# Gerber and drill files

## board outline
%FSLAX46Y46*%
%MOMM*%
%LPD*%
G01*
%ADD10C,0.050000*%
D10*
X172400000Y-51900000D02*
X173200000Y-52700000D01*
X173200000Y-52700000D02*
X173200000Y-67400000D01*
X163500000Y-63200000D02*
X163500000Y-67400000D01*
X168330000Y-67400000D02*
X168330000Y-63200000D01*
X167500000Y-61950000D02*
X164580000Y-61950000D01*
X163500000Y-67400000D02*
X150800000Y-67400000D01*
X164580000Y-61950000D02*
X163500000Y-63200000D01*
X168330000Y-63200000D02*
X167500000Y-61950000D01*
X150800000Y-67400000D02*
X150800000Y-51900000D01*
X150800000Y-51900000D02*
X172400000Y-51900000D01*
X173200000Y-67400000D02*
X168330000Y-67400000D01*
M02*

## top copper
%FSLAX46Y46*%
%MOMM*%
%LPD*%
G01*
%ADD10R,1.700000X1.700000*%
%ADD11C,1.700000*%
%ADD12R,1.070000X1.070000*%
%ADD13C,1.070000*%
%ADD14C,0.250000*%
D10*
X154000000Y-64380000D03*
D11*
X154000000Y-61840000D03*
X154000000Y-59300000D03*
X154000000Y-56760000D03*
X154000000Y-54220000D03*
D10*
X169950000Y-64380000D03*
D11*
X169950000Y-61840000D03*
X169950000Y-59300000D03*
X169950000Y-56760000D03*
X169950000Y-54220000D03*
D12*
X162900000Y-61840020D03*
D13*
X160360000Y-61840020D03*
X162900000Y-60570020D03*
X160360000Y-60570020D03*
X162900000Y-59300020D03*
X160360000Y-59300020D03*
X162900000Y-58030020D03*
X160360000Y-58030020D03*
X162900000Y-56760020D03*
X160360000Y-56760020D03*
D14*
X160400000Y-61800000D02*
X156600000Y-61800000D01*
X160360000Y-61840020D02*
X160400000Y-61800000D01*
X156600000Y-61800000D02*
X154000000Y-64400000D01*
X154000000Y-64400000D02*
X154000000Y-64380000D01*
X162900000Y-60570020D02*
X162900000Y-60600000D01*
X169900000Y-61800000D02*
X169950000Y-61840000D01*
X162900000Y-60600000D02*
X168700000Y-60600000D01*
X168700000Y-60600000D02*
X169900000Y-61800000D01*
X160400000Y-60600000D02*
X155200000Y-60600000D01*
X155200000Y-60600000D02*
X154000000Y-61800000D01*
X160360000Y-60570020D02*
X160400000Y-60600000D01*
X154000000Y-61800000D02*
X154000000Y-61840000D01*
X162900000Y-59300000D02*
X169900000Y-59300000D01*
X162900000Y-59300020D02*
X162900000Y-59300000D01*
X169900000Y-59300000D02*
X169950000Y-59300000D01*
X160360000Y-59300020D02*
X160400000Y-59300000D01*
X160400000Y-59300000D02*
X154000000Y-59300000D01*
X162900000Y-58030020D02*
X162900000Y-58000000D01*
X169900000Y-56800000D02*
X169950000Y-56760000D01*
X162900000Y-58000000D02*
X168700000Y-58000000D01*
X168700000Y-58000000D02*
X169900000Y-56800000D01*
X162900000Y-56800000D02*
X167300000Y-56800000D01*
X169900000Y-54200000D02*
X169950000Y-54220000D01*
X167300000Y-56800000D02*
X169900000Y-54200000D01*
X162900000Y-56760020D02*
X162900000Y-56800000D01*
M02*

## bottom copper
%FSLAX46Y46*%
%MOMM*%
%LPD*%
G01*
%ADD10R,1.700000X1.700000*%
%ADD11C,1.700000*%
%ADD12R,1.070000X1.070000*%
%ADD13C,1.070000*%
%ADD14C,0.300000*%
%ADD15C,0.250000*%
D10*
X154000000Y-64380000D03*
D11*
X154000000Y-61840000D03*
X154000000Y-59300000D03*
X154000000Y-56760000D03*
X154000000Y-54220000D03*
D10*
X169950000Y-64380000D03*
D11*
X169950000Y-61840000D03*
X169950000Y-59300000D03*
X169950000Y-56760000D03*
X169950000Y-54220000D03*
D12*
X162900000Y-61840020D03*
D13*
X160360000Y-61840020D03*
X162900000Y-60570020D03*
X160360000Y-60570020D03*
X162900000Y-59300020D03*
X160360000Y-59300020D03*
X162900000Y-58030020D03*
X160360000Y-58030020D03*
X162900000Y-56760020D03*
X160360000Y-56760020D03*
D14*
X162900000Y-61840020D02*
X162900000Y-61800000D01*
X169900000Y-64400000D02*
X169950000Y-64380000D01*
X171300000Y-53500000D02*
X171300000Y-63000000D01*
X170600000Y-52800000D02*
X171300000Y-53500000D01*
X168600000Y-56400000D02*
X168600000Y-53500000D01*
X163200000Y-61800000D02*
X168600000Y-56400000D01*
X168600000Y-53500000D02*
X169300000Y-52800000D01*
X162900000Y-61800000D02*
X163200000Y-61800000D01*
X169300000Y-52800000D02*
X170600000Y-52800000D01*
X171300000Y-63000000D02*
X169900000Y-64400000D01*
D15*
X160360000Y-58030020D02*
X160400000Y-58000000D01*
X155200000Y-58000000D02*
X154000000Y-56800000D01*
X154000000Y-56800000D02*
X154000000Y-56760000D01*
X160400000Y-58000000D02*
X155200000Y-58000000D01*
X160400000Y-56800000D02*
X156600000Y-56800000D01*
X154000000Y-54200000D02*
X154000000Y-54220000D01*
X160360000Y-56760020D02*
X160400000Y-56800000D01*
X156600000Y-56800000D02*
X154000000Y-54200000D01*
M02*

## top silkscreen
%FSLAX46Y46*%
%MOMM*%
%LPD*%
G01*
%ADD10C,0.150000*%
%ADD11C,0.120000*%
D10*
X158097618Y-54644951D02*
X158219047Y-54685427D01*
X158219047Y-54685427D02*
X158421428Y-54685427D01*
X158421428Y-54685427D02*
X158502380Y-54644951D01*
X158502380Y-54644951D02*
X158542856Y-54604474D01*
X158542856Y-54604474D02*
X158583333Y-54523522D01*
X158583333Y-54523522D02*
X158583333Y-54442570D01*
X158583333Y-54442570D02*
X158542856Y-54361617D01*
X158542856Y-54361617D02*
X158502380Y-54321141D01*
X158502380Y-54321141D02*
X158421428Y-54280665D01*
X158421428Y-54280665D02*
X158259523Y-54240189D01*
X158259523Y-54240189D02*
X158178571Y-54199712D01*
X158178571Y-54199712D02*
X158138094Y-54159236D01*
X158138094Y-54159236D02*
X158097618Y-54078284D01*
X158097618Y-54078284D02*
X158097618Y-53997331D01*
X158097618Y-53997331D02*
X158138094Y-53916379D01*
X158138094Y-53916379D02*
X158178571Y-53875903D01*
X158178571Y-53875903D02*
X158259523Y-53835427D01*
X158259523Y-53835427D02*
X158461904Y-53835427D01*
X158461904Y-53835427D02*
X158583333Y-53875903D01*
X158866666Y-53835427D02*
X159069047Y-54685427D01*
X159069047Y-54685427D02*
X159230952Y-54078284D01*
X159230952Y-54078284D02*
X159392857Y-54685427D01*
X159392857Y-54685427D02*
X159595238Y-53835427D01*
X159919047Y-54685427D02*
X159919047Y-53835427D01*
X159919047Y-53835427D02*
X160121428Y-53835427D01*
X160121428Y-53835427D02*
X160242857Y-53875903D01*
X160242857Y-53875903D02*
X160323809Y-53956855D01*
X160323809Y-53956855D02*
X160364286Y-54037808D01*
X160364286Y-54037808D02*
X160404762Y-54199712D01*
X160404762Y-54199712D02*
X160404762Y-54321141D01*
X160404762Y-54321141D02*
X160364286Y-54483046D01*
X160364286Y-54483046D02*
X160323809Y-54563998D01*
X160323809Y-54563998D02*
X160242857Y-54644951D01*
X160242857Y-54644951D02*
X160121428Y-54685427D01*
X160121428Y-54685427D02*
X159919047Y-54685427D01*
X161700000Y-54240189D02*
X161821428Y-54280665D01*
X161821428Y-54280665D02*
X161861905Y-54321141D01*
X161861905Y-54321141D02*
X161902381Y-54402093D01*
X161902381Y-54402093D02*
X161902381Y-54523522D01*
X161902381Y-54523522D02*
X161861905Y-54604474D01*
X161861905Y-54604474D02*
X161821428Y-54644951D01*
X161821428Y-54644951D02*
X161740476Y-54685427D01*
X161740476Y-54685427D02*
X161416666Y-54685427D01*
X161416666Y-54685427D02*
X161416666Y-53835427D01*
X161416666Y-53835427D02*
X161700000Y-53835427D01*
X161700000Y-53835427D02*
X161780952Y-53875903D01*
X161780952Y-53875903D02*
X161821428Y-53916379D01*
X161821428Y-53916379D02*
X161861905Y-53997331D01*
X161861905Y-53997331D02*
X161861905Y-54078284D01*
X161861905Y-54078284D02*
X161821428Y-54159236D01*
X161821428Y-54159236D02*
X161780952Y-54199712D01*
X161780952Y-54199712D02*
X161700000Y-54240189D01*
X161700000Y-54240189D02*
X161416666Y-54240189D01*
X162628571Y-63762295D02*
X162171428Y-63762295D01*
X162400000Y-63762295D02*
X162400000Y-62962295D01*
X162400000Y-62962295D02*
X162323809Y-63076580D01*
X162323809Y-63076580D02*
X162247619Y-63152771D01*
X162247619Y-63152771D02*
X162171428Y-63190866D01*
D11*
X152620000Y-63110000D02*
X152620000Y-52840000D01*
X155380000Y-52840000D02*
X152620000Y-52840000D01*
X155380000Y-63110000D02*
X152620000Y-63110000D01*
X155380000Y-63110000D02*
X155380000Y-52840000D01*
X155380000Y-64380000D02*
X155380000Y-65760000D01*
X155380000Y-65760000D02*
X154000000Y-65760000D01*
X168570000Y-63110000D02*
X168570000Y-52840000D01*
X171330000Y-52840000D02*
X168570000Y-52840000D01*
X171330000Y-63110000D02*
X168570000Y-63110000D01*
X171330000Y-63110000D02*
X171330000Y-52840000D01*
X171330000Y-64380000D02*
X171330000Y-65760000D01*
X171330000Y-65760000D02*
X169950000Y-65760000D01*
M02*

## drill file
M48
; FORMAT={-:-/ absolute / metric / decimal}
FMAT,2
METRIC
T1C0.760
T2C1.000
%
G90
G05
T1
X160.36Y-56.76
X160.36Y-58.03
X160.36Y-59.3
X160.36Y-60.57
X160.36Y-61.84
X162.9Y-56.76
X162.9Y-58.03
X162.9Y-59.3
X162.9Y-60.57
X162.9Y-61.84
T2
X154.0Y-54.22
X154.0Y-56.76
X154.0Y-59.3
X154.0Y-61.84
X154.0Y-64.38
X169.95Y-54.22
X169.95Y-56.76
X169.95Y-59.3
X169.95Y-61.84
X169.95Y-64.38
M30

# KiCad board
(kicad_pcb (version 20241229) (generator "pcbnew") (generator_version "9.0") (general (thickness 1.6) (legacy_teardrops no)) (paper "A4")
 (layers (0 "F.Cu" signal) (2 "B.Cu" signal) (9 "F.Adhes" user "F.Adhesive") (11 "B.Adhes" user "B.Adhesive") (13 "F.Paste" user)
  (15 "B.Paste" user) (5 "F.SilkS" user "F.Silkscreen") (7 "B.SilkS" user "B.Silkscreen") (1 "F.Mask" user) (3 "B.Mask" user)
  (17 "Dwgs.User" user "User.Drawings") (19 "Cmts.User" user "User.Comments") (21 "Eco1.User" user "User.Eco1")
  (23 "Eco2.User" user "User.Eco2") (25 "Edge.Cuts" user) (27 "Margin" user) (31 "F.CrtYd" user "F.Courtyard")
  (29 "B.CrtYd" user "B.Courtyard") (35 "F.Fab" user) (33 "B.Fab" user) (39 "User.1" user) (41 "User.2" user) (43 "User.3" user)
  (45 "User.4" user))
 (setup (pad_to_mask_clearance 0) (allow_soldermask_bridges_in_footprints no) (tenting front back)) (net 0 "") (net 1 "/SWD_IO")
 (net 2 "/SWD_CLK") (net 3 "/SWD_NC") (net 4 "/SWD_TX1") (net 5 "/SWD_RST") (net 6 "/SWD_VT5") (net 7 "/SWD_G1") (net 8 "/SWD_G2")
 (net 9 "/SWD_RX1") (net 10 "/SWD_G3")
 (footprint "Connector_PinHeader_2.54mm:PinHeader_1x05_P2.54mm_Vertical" (layer "F.Cu") (at 154 64.38 180)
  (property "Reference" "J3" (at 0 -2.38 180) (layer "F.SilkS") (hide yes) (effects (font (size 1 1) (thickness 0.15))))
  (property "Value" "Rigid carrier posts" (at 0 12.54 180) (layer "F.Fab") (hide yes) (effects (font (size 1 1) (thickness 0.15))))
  (fp_line (start 1.38 1.27) (end 1.38 11.54) (stroke (width 0.12) (type solid)) (layer "F.SilkS"))
  (fp_line (start -1.38 11.54) (end 1.38 11.54) (stroke (width 0.12) (type solid)) (layer "F.SilkS"))
  (fp_line (start -1.38 1.27) (end 1.38 1.27) (stroke (width 0.12) (type solid)) (layer "F.SilkS"))
  (fp_line (start -1.38 1.27) (end -1.38 11.54) (stroke (width 0.12) (type solid)) (layer "F.SilkS"))
  (fp_line (start -1.38 0) (end -1.38 -1.38) (stroke (width 0.12) (type solid)) (layer "F.SilkS"))
  (fp_line (start -1.38 -1.38) (end 0 -1.38) (stroke (width 0.12) (type solid)) (layer "F.SilkS"))
  (pad "1" thru_hole rect (at 0 0 180) (size 1.7 1.7) (drill 1) (layers "*.Cu" "*.Mask") (remove_unused_layers no) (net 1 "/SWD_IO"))
  (pad "2" thru_hole circle (at 0 2.54 180) (size 1.7 1.7) (drill 1) (layers "*.Cu" "*.Mask") (remove_unused_layers no) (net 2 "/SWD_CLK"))
  (pad "3" thru_hole circle (at 0 5.08 180) (size 1.7 1.7) (drill 1) (layers "*.Cu" "*.Mask") (remove_unused_layers no) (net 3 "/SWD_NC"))
  (pad "4" thru_hole circle (at 0 7.62 180) (size 1.7 1.7) (drill 1) (layers "*.Cu" "*.Mask") (remove_unused_layers no) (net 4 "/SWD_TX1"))
  (pad "5" thru_hole circle (at 0 10.16 180) (size 1.7 1.7) (drill 1) (layers "*.Cu" "*.Mask") (remove_unused_layers no) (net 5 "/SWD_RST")))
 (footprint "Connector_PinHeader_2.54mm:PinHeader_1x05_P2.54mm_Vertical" (layer "F.Cu") (at 169.95 64.38 180)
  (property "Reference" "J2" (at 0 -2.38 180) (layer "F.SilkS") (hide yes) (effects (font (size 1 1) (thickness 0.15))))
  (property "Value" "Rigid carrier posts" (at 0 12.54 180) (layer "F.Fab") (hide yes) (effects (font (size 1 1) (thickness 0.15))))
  (fp_line (start 1.38 1.27) (end 1.38 11.54) (stroke (width 0.12) (type solid)) (layer "F.SilkS"))
  (fp_line (start -1.38 11.54) (end 1.38 11.54) (stroke (width 0.12) (type solid)) (layer "F.SilkS"))
  (fp_line (start -1.38 1.27) (end 1.38 1.27) (stroke (width 0.12) (type solid)) (layer "F.SilkS"))
  (fp_line (start -1.38 1.27) (end -1.38 11.54) (stroke (width 0.12) (type solid)) (layer "F.SilkS"))
  (fp_line (start -1.38 0) (end -1.38 -1.38) (stroke (width 0.12) (type solid)) (layer "F.SilkS"))
  (fp_line (start -1.38 -1.38) (end 0 -1.38) (stroke (width 0.12) (type solid)) (layer "F.SilkS"))
  (pad "1" thru_hole rect (at 0 0 180) (size 1.7 1.7) (drill 1) (layers "*.Cu" "*.Mask") (remove_unused_layers no) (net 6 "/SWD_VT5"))
  (pad "2" thru_hole circle (at 0 2.54 180) (size 1.7 1.7) (drill 1) (layers "*.Cu" "*.Mask") (remove_unused_layers no) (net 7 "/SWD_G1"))
  (pad "3" thru_hole circle (at 0 5.08 180) (size 1.7 1.7) (drill 1) (layers "*.Cu" "*.Mask") (remove_unused_layers no) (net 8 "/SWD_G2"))
  (pad "4" thru_hole circle (at 0 7.62 180) (size 1.7 1.7) (drill 1) (layers "*.Cu" "*.Mask") (remove_unused_layers no) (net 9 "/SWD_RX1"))
  (pad "5" thru_hole circle (at 0 10.16 180) (size 1.7 1.7) (drill 1) (layers "*.Cu" "*.Mask") (remove_unused_layers no) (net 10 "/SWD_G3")))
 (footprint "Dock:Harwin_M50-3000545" (layer "B.Cu") (at 162.9 61.84002)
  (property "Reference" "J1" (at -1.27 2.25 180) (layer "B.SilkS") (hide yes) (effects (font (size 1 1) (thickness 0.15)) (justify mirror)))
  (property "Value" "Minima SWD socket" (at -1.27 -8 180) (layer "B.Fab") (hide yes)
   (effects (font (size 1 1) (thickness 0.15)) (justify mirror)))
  (pad "1" thru_hole rect (at 0 0) (size 1.07 1.07) (drill 0.76) (layers "*.Cu" "*.Mask") (remove_unused_layers no) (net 6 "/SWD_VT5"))
  (pad "2" thru_hole circle (at -2.54 0) (size 1.07 1.07) (drill 0.76) (layers "*.Cu" "*.Mask") (remove_unused_layers no) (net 1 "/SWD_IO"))
  (pad "3" thru_hole circle (at 0 -1.27) (size 1.07 1.07) (drill 0.76) (layers "*.Cu" "*.Mask") (remove_unused_layers no) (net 7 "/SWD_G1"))
  (pad "4" thru_hole circle (at -2.54 -1.27) (size 1.07 1.07) (drill 0.76) (layers "*.Cu" "*.Mask") (remove_unused_layers no)
   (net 2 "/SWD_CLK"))
  (pad "5" thru_hole circle (at 0 -2.54) (size 1.07 1.07) (drill 0.76) (layers "*.Cu" "*.Mask") (remove_unused_layers no) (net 8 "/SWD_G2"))
  (pad "6" thru_hole circle (at -2.54 -2.54) (size 1.07 1.07) (drill 0.76) (layers "*.Cu" "*.Mask") (remove_unused_layers no)
   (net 3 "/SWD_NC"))
  (pad "7" thru_hole circle (at 0 -3.81) (size 1.07 1.07) (drill 0.76) (layers "*.Cu" "*.Mask") (remove_unused_layers no) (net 9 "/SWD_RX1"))
  (pad "8" thru_hole circle (at -2.54 -3.81) (size 1.07 1.07) (drill 0.76) (layers "*.Cu" "*.Mask") (remove_unused_layers no)
   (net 4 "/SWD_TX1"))
  (pad "9" thru_hole circle (at 0 -5.08) (size 1.07 1.07) (drill 0.76) (layers "*.Cu" "*.Mask") (remove_unused_layers no) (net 10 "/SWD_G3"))
  (pad "10" thru_hole circle (at -2.54 -5.08) (size 1.07 1.07) (drill 0.76) (layers "*.Cu" "*.Mask") (remove_unused_layers no)
   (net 5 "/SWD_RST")))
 (gr_line (start 172.4 51.9) (end 173.2 52.7) (stroke (width 0.05) (type default)) (layer "Edge.Cuts"))
 (gr_line (start 173.2 52.7) (end 173.2 67.4) (stroke (width 0.05) (type default)) (layer "Edge.Cuts"))
 (gr_line (start 163.5 63.2) (end 163.5 67.4) (stroke (width 0.05) (type default)) (layer "Edge.Cuts"))
 (gr_line (start 168.33 67.4) (end 168.33 63.2) (stroke (width 0.05) (type default)) (layer "Edge.Cuts"))
 (gr_line (start 167.5 61.95) (end 164.58 61.95) (stroke (width 0.05) (type default)) (layer "Edge.Cuts"))
 (gr_line (start 163.5 67.4) (end 150.8 67.4) (stroke (width 0.05) (type default)) (layer "Edge.Cuts"))
 (gr_line (start 164.58 61.95) (end 163.5 63.2) (stroke (width 0.05) (type default)) (layer "Edge.Cuts"))
 (gr_line (start 168.33 63.2) (end 167.5 61.95) (stroke (width 0.05) (type default)) (layer "Edge.Cuts"))
 (gr_line (start 150.8 67.4) (end 150.8 51.9) (stroke (width 0.05) (type default)) (layer "Edge.Cuts"))
 (gr_line (start 150.8 51.9) (end 172.4 51.9) (stroke (width 0.05) (type default)) (layer "Edge.Cuts"))
 (gr_line (start 173.2 67.4) (end 168.33 67.4) (stroke (width 0.05) (type default)) (layer "Edge.Cuts"))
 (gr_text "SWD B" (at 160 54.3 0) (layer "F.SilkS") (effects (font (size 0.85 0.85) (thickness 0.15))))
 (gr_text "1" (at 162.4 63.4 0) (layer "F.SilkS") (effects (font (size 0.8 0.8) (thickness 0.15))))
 (segment (start 162.9 61.84002) (end 162.9 61.8) (width 0.3) (layer "B.Cu") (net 6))
 (segment (start 169.9 64.4) (end 169.95 64.38) (width 0.3) (layer "B.Cu") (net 6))
 (segment (start 171.3 53.5) (end 171.3 63) (width 0.3) (layer "B.Cu") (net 6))
 (segment (start 170.6 52.8) (end 171.3 53.5) (width 0.3) (layer "B.Cu") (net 6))
 (segment (start 168.6 56.4) (end 168.6 53.5) (width 0.3) (layer "B.Cu") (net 6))
 (segment (start 163.2 61.8) (end 168.6 56.4) (width 0.3) (layer "B.Cu") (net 6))
 (segment (start 168.6 53.5) (end 169.3 52.8) (width 0.3) (layer "B.Cu") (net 6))
 (segment (start 162.9 61.8) (end 163.2 61.8) (width 0.3) (layer "B.Cu") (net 6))
 (segment (start 169.3 52.8) (end 170.6 52.8) (width 0.3) (layer "B.Cu") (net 6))
 (segment (start 171.3 63) (end 169.9 64.4) (width 0.3) (layer "B.Cu") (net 6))
 (segment (start 160.4 61.8) (end 156.6 61.8) (width 0.25) (layer "F.Cu") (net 1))
 (segment (start 160.36 61.84002) (end 160.4 61.8) (width 0.25) (layer "F.Cu") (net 1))
 (segment (start 156.6 61.8) (end 154 64.4) (width 0.25) (layer "F.Cu") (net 1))
 (segment (start 154 64.4) (end 154 64.38) (width 0.25) (layer "F.Cu") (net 1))
 (segment (start 162.9 60.57002) (end 162.9 60.6) (width 0.25) (layer "F.Cu") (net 7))
 (segment (start 169.9 61.8) (end 169.95 61.84) (width 0.25) (layer "F.Cu") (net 7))
 (segment (start 162.9 60.6) (end 168.7 60.6) (width 0.25) (layer "F.Cu") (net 7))
 (segment (start 168.7 60.6) (end 169.9 61.8) (width 0.25) (layer "F.Cu") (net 7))
 (segment (start 160.4 60.6) (end 155.2 60.6) (width 0.25) (layer "F.Cu") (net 2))
 (segment (start 155.2 60.6) (end 154 61.8) (width 0.25) (layer "F.Cu") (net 2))
 (segment (start 160.36 60.57002) (end 160.4 60.6) (width 0.25) (layer "F.Cu") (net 2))
 (segment (start 154 61.8) (end 154 61.84) (width 0.25) (layer "F.Cu") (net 2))
 (segment (start 162.9 59.3) (end 169.9 59.3) (width 0.25) (layer "F.Cu") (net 8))
 (segment (start 162.9 59.30002) (end 162.9 59.3) (width 0.25) (layer "F.Cu") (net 8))
 (segment (start 169.9 59.3) (end 169.95 59.3) (width 0.25) (layer "F.Cu") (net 8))
 (segment (start 160.36 59.30002) (end 160.4 59.3) (width 0.25) (layer "F.Cu") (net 3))
 (segment (start 160.4 59.3) (end 154 59.3) (width 0.25) (layer "F.Cu") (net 3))
 (segment (start 162.9 58.03002) (end 162.9 58) (width 0.25) (layer "F.Cu") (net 9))
 (segment (start 169.9 56.8) (end 169.95 56.76) (width 0.25) (layer "F.Cu") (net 9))
 (segment (start 162.9 58) (end 168.7 58) (width 0.25) (layer "F.Cu") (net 9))
 (segment (start 168.7 58) (end 169.9 56.8) (width 0.25) (layer "F.Cu") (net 9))
 (segment (start 160.36 58.03002) (end 160.4 58) (width 0.25) (layer "B.Cu") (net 4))
 (segment (start 155.2 58) (end 154 56.8) (width 0.25) (layer "B.Cu") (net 4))
 (segment (start 154 56.8) (end 154 56.76) (width 0.25) (layer "B.Cu") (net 4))
 (segment (start 160.4 58) (end 155.2 58) (width 0.25) (layer "B.Cu") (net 4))
 (segment (start 162.9 56.8) (end 167.3 56.8) (width 0.25) (layer "F.Cu") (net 10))
 (segment (start 169.9 54.2) (end 169.95 54.22) (width 0.25) (layer "F.Cu") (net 10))
 (segment (start 167.3 56.8) (end 169.9 54.2) (width 0.25) (layer "F.Cu") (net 10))
 (segment (start 162.9 56.76002) (end 162.9 56.8) (width 0.25) (layer "F.Cu") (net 10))
 (segment (start 160.4 56.8) (end 156.6 56.8) (width 0.25) (layer "B.Cu") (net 5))
 (segment (start 154 54.2) (end 154 54.22) (width 0.25) (layer "B.Cu") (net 5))
 (segment (start 160.36 56.76002) (end 160.4 56.8) (width 0.25) (layer "B.Cu") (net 5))
 (segment (start 156.6 56.8) (end 154 54.2) (width 0.25) (layer "B.Cu") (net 5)))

